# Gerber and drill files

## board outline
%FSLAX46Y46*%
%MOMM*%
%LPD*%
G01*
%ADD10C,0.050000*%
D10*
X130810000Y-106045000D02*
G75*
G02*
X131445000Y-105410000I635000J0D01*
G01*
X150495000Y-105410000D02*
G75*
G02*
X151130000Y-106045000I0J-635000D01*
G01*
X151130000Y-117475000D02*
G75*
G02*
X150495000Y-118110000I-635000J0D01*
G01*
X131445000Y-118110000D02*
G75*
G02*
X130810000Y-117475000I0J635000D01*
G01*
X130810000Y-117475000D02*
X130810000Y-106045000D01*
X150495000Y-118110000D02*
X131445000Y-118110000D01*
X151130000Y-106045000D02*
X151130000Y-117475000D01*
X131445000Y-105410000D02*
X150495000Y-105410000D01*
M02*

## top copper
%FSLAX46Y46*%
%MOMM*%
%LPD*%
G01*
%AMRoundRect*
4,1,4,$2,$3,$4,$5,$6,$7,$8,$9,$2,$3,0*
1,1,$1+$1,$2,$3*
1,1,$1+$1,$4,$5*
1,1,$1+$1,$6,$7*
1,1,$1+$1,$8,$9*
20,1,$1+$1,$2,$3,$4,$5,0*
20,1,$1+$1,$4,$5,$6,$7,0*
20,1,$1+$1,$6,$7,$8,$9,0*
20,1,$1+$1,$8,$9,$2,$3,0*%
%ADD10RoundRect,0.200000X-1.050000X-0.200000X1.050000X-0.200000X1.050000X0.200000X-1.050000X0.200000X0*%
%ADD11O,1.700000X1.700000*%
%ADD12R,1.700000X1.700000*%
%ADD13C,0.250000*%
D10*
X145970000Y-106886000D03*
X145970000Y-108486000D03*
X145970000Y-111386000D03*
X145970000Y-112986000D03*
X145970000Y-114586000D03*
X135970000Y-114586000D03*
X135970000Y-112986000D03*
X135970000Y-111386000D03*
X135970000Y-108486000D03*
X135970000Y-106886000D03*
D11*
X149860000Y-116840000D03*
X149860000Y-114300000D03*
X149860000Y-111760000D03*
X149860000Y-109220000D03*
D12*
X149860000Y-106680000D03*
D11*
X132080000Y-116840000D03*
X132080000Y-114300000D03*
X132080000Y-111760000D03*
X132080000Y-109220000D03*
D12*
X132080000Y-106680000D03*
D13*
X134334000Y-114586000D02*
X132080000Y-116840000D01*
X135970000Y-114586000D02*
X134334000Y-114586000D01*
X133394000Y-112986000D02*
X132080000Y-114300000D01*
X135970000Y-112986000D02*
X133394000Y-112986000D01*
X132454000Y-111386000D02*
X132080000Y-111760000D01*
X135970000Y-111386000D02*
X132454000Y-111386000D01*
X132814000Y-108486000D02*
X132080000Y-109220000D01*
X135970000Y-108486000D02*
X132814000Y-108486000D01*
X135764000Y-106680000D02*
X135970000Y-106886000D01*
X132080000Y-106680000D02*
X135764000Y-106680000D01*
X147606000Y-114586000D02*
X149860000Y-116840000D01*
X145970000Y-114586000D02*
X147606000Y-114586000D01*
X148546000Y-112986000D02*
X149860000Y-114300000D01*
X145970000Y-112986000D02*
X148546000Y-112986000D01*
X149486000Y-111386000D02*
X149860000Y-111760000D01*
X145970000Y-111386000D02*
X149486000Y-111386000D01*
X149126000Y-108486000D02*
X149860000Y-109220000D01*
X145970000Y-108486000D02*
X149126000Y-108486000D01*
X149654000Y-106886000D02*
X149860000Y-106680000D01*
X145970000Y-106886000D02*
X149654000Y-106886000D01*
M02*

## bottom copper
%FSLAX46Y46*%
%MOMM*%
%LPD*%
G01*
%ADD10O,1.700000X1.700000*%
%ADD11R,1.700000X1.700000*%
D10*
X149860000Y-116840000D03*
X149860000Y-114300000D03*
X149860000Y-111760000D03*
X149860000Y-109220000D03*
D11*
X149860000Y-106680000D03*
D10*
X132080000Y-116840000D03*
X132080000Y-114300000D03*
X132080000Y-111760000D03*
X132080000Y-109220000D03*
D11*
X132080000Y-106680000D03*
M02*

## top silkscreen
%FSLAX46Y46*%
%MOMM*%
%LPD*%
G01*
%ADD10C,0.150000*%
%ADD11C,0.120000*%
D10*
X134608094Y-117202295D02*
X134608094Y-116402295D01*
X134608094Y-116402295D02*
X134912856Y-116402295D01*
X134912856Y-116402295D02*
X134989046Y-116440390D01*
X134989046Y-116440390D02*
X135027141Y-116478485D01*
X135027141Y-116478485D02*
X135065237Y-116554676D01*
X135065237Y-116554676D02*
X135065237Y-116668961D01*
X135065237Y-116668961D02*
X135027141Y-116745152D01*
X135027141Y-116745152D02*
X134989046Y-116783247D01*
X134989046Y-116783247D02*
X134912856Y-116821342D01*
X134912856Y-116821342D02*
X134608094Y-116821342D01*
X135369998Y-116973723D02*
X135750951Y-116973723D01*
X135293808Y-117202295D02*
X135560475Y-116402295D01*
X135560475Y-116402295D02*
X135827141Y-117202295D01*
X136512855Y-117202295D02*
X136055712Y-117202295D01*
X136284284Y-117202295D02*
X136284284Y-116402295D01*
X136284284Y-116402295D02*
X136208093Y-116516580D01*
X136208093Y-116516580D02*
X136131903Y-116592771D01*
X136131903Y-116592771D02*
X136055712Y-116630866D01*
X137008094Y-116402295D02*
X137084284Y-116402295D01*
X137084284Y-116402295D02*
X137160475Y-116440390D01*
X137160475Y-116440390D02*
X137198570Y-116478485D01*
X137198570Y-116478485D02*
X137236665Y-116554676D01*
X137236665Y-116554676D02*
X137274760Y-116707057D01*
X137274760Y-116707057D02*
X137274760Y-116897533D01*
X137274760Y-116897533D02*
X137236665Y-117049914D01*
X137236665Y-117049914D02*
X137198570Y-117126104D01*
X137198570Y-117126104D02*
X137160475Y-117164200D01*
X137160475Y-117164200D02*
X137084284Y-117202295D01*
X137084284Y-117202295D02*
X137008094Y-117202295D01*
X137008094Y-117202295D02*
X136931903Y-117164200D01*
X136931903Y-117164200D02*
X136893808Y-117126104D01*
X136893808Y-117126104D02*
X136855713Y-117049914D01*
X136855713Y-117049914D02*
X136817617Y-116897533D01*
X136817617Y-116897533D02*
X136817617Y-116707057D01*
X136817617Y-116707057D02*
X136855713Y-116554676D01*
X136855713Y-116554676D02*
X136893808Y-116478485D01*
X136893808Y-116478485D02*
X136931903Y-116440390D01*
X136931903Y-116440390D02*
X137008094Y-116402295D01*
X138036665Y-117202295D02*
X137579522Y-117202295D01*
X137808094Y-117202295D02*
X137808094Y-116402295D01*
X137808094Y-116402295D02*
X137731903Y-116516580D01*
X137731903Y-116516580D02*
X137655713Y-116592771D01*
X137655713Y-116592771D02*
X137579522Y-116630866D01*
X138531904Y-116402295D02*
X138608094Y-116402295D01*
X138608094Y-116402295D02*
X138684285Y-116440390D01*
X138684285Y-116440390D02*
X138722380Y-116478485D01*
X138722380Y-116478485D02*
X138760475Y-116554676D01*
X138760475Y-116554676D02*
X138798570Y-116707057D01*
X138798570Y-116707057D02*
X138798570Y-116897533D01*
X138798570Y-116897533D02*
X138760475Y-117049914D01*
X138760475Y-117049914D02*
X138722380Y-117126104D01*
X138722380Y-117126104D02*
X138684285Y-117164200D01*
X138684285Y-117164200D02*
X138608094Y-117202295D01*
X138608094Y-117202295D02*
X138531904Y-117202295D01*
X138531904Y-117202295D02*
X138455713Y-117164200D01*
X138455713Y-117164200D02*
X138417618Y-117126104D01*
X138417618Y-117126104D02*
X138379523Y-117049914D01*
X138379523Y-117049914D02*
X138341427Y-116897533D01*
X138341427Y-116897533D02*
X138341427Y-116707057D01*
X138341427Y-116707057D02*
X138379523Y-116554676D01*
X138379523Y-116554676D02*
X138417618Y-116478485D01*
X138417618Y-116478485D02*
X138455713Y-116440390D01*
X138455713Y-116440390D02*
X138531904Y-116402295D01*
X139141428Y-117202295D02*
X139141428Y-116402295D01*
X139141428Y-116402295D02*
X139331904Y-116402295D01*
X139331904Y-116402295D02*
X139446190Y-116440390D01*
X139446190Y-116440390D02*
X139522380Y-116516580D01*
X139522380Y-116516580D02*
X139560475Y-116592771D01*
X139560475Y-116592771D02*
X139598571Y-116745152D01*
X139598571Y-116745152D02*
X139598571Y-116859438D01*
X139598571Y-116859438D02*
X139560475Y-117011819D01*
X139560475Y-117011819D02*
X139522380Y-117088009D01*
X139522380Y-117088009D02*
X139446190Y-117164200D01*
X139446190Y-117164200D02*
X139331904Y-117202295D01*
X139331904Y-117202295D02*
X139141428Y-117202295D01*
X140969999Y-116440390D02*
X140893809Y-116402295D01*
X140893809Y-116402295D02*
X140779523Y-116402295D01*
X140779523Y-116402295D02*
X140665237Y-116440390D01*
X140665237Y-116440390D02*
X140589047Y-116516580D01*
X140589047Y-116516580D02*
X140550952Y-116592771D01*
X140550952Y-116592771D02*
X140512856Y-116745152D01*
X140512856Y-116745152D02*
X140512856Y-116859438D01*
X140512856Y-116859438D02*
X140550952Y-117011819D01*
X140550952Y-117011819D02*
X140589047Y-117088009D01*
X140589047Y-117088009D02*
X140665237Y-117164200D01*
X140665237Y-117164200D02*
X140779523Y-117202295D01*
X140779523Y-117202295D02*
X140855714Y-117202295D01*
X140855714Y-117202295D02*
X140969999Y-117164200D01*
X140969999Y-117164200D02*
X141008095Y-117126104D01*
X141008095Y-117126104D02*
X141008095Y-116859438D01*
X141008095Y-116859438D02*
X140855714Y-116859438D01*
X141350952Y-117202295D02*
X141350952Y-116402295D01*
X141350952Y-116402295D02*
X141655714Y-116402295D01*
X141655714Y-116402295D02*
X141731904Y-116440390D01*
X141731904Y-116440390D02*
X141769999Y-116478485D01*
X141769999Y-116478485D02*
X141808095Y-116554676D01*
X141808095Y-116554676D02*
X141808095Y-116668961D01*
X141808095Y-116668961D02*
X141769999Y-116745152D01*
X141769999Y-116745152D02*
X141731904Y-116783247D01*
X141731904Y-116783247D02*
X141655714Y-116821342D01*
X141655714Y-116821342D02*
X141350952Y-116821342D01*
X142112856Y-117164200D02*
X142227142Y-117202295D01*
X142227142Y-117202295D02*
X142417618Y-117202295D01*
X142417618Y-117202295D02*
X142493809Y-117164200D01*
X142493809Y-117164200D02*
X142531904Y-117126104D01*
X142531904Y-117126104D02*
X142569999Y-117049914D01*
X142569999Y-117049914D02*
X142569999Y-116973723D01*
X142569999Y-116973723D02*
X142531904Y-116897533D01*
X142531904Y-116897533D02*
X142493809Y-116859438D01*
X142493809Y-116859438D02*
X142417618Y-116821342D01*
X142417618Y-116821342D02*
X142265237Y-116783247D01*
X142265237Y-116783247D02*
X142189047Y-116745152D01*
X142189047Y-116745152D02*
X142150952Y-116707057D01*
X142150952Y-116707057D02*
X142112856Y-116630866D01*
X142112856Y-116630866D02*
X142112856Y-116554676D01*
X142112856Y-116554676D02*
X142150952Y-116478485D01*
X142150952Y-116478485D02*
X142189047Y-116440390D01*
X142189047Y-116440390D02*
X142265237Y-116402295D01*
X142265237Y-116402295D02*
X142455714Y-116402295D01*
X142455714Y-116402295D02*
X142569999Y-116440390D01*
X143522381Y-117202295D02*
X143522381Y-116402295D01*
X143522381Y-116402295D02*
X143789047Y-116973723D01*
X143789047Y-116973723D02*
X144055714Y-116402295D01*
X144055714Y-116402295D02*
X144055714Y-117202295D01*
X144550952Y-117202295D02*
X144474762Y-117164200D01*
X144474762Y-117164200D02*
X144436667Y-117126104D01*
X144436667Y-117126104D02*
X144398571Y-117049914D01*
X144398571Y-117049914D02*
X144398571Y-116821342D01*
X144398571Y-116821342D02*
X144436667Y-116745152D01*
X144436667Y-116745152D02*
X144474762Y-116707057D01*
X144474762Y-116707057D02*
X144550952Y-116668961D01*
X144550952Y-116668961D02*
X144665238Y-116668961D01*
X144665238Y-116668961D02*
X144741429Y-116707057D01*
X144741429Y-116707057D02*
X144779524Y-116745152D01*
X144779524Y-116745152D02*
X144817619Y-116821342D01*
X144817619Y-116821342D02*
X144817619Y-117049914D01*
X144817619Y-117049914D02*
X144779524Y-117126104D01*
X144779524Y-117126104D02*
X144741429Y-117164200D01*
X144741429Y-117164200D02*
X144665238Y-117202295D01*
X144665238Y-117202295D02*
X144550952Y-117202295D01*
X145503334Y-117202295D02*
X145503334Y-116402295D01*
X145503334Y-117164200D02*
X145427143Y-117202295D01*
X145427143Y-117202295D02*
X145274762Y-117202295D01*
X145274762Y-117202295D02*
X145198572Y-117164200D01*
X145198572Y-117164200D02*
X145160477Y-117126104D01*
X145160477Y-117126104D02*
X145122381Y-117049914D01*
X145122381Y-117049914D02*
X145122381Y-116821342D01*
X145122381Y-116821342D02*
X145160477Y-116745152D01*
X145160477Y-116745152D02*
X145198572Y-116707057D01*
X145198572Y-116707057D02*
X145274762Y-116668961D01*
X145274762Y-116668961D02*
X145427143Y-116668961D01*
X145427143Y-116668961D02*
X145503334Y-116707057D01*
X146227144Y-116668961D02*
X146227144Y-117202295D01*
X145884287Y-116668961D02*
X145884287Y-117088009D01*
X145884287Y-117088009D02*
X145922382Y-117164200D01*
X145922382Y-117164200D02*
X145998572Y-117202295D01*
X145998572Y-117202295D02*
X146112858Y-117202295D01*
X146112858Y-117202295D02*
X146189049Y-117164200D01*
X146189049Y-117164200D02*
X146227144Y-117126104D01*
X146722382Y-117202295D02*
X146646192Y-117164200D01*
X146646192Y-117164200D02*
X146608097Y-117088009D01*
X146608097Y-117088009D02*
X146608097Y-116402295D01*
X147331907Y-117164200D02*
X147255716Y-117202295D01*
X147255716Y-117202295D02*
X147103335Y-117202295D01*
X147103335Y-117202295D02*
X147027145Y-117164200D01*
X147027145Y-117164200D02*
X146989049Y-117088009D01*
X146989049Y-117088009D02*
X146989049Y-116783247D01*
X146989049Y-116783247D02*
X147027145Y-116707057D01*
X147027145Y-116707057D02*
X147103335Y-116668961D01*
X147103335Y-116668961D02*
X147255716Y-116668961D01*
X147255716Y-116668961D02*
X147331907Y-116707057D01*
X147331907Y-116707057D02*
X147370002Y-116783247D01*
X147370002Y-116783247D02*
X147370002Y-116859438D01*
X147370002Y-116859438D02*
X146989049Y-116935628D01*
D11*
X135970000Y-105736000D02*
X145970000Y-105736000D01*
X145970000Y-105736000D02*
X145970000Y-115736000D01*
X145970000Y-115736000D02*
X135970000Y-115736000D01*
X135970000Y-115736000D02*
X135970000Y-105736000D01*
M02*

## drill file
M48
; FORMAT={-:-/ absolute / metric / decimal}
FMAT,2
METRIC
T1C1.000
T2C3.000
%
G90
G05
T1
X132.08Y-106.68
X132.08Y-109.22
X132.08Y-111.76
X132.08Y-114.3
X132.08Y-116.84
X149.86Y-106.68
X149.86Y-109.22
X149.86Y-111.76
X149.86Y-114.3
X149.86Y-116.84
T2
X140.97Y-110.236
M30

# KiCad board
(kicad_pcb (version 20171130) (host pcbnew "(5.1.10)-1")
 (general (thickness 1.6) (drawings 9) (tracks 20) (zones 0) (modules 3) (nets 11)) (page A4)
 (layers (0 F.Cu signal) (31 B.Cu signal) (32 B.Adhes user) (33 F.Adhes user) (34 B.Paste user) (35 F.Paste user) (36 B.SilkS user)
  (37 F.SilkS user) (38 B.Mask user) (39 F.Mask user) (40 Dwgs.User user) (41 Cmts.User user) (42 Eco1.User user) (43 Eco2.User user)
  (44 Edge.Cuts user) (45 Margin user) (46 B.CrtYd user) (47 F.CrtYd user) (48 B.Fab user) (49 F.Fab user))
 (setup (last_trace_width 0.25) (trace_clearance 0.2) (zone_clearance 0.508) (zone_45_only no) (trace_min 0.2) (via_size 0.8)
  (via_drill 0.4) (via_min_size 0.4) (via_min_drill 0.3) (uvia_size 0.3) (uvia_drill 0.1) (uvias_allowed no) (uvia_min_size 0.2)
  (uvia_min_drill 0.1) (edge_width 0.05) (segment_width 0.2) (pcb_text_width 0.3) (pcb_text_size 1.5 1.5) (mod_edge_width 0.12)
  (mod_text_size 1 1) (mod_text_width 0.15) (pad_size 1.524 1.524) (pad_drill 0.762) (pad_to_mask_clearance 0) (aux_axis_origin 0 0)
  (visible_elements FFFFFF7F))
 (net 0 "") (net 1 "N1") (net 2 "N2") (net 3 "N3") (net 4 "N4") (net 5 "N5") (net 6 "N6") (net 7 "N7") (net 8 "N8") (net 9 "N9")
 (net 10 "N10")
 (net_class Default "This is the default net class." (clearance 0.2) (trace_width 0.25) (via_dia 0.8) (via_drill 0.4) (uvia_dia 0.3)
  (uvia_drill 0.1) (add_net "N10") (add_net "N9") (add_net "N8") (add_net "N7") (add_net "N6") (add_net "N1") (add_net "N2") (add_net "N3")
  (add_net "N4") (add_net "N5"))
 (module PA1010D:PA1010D (layer F.Cu) (at 140.97 110.736)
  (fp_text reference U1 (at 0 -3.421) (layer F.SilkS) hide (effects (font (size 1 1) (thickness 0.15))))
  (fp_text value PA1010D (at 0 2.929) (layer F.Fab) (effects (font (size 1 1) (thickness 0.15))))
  (fp_line (start -5 -5) (end 5 -5) (layer F.SilkS) (width 0.12))
  (fp_line (start 5 -5) (end 5 5) (layer F.SilkS) (width 0.12))
  (fp_line (start 5 5) (end -5 5) (layer F.SilkS) (width 0.12))
  (fp_line (start -5 5) (end -5 -5) (layer F.SilkS) (width 0.12))
  (pad "" np_thru_hole circle (at 0 -0.5) (size 3 3) (drill 3) (layers *.Cu *.Mask))
  (pad 10 smd roundrect (at 5 -3.85) (size 2.5 0.8) (layers F.Cu F.Paste F.Mask) (roundrect_rratio 0.25) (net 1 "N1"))
  (pad 9 smd roundrect (at 5 -2.25) (size 2.5 0.8) (layers F.Cu F.Paste F.Mask) (roundrect_rratio 0.25) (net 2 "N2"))
  (pad 8 smd roundrect (at 5 0.65) (size 2.5 0.8) (layers F.Cu F.Paste F.Mask) (roundrect_rratio 0.25) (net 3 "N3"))
  (pad 7 smd roundrect (at 5 2.25) (size 2.5 0.8) (layers F.Cu F.Paste F.Mask) (roundrect_rratio 0.25) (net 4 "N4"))
  (pad 6 smd roundrect (at 5 3.85) (size 2.5 0.8) (layers F.Cu F.Paste F.Mask) (roundrect_rratio 0.25) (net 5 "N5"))
  (pad 5 smd roundrect (at -5 3.85) (size 2.5 0.8) (layers F.Cu F.Paste F.Mask) (roundrect_rratio 0.25) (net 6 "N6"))
  (pad 4 smd roundrect (at -5 2.25) (size 2.5 0.8) (layers F.Cu F.Paste F.Mask) (roundrect_rratio 0.25) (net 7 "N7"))
  (pad 3 smd roundrect (at -5 0.65) (size 2.5 0.8) (layers F.Cu F.Paste F.Mask) (roundrect_rratio 0.25) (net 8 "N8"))
  (pad 2 smd roundrect (at -5 -2.25) (size 2.5 0.8) (layers F.Cu F.Paste F.Mask) (roundrect_rratio 0.25) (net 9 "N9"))
  (pad 1 smd roundrect (at -5 -3.85) (size 2.5 0.8) (layers F.Cu F.Paste F.Mask) (roundrect_rratio 0.25) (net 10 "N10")))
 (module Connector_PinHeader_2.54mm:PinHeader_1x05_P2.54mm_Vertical (layer B.Cu) (at 149.86 106.68 180)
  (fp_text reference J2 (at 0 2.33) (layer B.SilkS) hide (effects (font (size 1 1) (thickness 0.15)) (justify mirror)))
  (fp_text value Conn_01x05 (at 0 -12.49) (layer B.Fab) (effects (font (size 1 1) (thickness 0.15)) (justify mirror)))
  (pad 5 thru_hole oval (at 0 -10.16 180) (size 1.7 1.7) (drill 1) (layers *.Cu *.Mask) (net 5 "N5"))
  (pad 4 thru_hole oval (at 0 -7.62 180) (size 1.7 1.7) (drill 1) (layers *.Cu *.Mask) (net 4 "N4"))
  (pad 3 thru_hole oval (at 0 -5.08 180) (size 1.7 1.7) (drill 1) (layers *.Cu *.Mask) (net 3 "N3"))
  (pad 2 thru_hole oval (at 0 -2.54 180) (size 1.7 1.7) (drill 1) (layers *.Cu *.Mask) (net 2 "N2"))
  (pad 1 thru_hole rect (at 0 0 180) (size 1.7 1.7) (drill 1) (layers *.Cu *.Mask) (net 1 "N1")))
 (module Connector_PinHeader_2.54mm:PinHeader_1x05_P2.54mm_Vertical (layer B.Cu) (at 132.08 106.68 180)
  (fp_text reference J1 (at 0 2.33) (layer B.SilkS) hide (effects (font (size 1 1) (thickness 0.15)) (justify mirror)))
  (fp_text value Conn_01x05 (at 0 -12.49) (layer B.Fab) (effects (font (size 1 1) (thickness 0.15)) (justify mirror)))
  (pad 5 thru_hole oval (at 0 -10.16 180) (size 1.7 1.7) (drill 1) (layers *.Cu *.Mask) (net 6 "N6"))
  (pad 4 thru_hole oval (at 0 -7.62 180) (size 1.7 1.7) (drill 1) (layers *.Cu *.Mask) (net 7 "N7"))
  (pad 3 thru_hole oval (at 0 -5.08 180) (size 1.7 1.7) (drill 1) (layers *.Cu *.Mask) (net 8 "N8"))
  (pad 2 thru_hole oval (at 0 -2.54 180) (size 1.7 1.7) (drill 1) (layers *.Cu *.Mask) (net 9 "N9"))
  (pad 1 thru_hole rect (at 0 0 180) (size 1.7 1.7) (drill 1) (layers *.Cu *.Mask) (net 10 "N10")))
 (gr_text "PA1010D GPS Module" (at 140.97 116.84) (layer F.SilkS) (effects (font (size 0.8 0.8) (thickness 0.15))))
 (gr_arc (start 131.445 106.045) (end 131.445 105.41) (angle -90) (layer Edge.Cuts) (width 0.05))
 (gr_arc (start 150.495 106.045) (end 151.13 106.045) (angle -90) (layer Edge.Cuts) (width 0.05))
 (gr_arc (start 150.495 117.475) (end 150.495 118.11) (angle -90) (layer Edge.Cuts) (width 0.05))
 (gr_arc (start 131.445 117.475) (end 130.81 117.475) (angle -90) (layer Edge.Cuts) (width 0.05))
 (gr_line (start 130.81 117.475) (end 130.81 106.045) (layer Edge.Cuts) (width 0.05))
 (gr_line (start 150.495 118.11) (end 131.445 118.11) (layer Edge.Cuts) (width 0.05))
 (gr_line (start 151.13 106.045) (end 151.13 117.475) (layer Edge.Cuts) (width 0.05))
 (gr_line (start 131.445 105.41) (end 150.495 105.41) (layer Edge.Cuts) (width 0.05))
 (segment (start 134.334 114.586) (end 132.08 116.84) (width 0.25) (layer F.Cu) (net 6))
 (segment (start 135.97 114.586) (end 134.334 114.586) (width 0.25) (layer F.Cu) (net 6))
 (segment (start 133.394 112.986) (end 132.08 114.3) (width 0.25) (layer F.Cu) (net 7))
 (segment (start 135.97 112.986) (end 133.394 112.986) (width 0.25) (layer F.Cu) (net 7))
 (segment (start 132.454 111.386) (end 132.08 111.76) (width 0.25) (layer F.Cu) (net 8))
 (segment (start 135.97 111.386) (end 132.454 111.386) (width 0.25) (layer F.Cu) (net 8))
 (segment (start 132.814 108.486) (end 132.08 109.22) (width 0.25) (layer F.Cu) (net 9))
 (segment (start 135.97 108.486) (end 132.814 108.486) (width 0.25) (layer F.Cu) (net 9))
 (segment (start 135.764 106.68) (end 135.97 106.886) (width 0.25) (layer F.Cu) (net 10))
 (segment (start 132.08 106.68) (end 135.764 106.68) (width 0.25) (layer F.Cu) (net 10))
 (segment (start 147.606 114.586) (end 149.86 116.84) (width 0.25) (layer F.Cu) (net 5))
 (segment (start 145.97 114.586) (end 147.606 114.586) (width 0.25) (layer F.Cu) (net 5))
 (segment (start 148.546 112.986) (end 149.86 114.3) (width 0.25) (layer F.Cu) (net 4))
 (segment (start 145.97 112.986) (end 148.546 112.986) (width 0.25) (layer F.Cu) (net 4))
 (segment (start 149.486 111.386) (end 149.86 111.76) (width 0.25) (layer F.Cu) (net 3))
 (segment (start 145.97 111.386) (end 149.486 111.386) (width 0.25) (layer F.Cu) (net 3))
 (segment (start 149.126 108.486) (end 149.86 109.22) (width 0.25) (layer F.Cu) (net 2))
 (segment (start 145.97 108.486) (end 149.126 108.486) (width 0.25) (layer F.Cu) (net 2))
 (segment (start 149.654 106.886) (end 149.86 106.68) (width 0.25) (layer F.Cu) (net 1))
 (segment (start 145.97 106.886) (end 149.654 106.886) (width 0.25) (layer F.Cu) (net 1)))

